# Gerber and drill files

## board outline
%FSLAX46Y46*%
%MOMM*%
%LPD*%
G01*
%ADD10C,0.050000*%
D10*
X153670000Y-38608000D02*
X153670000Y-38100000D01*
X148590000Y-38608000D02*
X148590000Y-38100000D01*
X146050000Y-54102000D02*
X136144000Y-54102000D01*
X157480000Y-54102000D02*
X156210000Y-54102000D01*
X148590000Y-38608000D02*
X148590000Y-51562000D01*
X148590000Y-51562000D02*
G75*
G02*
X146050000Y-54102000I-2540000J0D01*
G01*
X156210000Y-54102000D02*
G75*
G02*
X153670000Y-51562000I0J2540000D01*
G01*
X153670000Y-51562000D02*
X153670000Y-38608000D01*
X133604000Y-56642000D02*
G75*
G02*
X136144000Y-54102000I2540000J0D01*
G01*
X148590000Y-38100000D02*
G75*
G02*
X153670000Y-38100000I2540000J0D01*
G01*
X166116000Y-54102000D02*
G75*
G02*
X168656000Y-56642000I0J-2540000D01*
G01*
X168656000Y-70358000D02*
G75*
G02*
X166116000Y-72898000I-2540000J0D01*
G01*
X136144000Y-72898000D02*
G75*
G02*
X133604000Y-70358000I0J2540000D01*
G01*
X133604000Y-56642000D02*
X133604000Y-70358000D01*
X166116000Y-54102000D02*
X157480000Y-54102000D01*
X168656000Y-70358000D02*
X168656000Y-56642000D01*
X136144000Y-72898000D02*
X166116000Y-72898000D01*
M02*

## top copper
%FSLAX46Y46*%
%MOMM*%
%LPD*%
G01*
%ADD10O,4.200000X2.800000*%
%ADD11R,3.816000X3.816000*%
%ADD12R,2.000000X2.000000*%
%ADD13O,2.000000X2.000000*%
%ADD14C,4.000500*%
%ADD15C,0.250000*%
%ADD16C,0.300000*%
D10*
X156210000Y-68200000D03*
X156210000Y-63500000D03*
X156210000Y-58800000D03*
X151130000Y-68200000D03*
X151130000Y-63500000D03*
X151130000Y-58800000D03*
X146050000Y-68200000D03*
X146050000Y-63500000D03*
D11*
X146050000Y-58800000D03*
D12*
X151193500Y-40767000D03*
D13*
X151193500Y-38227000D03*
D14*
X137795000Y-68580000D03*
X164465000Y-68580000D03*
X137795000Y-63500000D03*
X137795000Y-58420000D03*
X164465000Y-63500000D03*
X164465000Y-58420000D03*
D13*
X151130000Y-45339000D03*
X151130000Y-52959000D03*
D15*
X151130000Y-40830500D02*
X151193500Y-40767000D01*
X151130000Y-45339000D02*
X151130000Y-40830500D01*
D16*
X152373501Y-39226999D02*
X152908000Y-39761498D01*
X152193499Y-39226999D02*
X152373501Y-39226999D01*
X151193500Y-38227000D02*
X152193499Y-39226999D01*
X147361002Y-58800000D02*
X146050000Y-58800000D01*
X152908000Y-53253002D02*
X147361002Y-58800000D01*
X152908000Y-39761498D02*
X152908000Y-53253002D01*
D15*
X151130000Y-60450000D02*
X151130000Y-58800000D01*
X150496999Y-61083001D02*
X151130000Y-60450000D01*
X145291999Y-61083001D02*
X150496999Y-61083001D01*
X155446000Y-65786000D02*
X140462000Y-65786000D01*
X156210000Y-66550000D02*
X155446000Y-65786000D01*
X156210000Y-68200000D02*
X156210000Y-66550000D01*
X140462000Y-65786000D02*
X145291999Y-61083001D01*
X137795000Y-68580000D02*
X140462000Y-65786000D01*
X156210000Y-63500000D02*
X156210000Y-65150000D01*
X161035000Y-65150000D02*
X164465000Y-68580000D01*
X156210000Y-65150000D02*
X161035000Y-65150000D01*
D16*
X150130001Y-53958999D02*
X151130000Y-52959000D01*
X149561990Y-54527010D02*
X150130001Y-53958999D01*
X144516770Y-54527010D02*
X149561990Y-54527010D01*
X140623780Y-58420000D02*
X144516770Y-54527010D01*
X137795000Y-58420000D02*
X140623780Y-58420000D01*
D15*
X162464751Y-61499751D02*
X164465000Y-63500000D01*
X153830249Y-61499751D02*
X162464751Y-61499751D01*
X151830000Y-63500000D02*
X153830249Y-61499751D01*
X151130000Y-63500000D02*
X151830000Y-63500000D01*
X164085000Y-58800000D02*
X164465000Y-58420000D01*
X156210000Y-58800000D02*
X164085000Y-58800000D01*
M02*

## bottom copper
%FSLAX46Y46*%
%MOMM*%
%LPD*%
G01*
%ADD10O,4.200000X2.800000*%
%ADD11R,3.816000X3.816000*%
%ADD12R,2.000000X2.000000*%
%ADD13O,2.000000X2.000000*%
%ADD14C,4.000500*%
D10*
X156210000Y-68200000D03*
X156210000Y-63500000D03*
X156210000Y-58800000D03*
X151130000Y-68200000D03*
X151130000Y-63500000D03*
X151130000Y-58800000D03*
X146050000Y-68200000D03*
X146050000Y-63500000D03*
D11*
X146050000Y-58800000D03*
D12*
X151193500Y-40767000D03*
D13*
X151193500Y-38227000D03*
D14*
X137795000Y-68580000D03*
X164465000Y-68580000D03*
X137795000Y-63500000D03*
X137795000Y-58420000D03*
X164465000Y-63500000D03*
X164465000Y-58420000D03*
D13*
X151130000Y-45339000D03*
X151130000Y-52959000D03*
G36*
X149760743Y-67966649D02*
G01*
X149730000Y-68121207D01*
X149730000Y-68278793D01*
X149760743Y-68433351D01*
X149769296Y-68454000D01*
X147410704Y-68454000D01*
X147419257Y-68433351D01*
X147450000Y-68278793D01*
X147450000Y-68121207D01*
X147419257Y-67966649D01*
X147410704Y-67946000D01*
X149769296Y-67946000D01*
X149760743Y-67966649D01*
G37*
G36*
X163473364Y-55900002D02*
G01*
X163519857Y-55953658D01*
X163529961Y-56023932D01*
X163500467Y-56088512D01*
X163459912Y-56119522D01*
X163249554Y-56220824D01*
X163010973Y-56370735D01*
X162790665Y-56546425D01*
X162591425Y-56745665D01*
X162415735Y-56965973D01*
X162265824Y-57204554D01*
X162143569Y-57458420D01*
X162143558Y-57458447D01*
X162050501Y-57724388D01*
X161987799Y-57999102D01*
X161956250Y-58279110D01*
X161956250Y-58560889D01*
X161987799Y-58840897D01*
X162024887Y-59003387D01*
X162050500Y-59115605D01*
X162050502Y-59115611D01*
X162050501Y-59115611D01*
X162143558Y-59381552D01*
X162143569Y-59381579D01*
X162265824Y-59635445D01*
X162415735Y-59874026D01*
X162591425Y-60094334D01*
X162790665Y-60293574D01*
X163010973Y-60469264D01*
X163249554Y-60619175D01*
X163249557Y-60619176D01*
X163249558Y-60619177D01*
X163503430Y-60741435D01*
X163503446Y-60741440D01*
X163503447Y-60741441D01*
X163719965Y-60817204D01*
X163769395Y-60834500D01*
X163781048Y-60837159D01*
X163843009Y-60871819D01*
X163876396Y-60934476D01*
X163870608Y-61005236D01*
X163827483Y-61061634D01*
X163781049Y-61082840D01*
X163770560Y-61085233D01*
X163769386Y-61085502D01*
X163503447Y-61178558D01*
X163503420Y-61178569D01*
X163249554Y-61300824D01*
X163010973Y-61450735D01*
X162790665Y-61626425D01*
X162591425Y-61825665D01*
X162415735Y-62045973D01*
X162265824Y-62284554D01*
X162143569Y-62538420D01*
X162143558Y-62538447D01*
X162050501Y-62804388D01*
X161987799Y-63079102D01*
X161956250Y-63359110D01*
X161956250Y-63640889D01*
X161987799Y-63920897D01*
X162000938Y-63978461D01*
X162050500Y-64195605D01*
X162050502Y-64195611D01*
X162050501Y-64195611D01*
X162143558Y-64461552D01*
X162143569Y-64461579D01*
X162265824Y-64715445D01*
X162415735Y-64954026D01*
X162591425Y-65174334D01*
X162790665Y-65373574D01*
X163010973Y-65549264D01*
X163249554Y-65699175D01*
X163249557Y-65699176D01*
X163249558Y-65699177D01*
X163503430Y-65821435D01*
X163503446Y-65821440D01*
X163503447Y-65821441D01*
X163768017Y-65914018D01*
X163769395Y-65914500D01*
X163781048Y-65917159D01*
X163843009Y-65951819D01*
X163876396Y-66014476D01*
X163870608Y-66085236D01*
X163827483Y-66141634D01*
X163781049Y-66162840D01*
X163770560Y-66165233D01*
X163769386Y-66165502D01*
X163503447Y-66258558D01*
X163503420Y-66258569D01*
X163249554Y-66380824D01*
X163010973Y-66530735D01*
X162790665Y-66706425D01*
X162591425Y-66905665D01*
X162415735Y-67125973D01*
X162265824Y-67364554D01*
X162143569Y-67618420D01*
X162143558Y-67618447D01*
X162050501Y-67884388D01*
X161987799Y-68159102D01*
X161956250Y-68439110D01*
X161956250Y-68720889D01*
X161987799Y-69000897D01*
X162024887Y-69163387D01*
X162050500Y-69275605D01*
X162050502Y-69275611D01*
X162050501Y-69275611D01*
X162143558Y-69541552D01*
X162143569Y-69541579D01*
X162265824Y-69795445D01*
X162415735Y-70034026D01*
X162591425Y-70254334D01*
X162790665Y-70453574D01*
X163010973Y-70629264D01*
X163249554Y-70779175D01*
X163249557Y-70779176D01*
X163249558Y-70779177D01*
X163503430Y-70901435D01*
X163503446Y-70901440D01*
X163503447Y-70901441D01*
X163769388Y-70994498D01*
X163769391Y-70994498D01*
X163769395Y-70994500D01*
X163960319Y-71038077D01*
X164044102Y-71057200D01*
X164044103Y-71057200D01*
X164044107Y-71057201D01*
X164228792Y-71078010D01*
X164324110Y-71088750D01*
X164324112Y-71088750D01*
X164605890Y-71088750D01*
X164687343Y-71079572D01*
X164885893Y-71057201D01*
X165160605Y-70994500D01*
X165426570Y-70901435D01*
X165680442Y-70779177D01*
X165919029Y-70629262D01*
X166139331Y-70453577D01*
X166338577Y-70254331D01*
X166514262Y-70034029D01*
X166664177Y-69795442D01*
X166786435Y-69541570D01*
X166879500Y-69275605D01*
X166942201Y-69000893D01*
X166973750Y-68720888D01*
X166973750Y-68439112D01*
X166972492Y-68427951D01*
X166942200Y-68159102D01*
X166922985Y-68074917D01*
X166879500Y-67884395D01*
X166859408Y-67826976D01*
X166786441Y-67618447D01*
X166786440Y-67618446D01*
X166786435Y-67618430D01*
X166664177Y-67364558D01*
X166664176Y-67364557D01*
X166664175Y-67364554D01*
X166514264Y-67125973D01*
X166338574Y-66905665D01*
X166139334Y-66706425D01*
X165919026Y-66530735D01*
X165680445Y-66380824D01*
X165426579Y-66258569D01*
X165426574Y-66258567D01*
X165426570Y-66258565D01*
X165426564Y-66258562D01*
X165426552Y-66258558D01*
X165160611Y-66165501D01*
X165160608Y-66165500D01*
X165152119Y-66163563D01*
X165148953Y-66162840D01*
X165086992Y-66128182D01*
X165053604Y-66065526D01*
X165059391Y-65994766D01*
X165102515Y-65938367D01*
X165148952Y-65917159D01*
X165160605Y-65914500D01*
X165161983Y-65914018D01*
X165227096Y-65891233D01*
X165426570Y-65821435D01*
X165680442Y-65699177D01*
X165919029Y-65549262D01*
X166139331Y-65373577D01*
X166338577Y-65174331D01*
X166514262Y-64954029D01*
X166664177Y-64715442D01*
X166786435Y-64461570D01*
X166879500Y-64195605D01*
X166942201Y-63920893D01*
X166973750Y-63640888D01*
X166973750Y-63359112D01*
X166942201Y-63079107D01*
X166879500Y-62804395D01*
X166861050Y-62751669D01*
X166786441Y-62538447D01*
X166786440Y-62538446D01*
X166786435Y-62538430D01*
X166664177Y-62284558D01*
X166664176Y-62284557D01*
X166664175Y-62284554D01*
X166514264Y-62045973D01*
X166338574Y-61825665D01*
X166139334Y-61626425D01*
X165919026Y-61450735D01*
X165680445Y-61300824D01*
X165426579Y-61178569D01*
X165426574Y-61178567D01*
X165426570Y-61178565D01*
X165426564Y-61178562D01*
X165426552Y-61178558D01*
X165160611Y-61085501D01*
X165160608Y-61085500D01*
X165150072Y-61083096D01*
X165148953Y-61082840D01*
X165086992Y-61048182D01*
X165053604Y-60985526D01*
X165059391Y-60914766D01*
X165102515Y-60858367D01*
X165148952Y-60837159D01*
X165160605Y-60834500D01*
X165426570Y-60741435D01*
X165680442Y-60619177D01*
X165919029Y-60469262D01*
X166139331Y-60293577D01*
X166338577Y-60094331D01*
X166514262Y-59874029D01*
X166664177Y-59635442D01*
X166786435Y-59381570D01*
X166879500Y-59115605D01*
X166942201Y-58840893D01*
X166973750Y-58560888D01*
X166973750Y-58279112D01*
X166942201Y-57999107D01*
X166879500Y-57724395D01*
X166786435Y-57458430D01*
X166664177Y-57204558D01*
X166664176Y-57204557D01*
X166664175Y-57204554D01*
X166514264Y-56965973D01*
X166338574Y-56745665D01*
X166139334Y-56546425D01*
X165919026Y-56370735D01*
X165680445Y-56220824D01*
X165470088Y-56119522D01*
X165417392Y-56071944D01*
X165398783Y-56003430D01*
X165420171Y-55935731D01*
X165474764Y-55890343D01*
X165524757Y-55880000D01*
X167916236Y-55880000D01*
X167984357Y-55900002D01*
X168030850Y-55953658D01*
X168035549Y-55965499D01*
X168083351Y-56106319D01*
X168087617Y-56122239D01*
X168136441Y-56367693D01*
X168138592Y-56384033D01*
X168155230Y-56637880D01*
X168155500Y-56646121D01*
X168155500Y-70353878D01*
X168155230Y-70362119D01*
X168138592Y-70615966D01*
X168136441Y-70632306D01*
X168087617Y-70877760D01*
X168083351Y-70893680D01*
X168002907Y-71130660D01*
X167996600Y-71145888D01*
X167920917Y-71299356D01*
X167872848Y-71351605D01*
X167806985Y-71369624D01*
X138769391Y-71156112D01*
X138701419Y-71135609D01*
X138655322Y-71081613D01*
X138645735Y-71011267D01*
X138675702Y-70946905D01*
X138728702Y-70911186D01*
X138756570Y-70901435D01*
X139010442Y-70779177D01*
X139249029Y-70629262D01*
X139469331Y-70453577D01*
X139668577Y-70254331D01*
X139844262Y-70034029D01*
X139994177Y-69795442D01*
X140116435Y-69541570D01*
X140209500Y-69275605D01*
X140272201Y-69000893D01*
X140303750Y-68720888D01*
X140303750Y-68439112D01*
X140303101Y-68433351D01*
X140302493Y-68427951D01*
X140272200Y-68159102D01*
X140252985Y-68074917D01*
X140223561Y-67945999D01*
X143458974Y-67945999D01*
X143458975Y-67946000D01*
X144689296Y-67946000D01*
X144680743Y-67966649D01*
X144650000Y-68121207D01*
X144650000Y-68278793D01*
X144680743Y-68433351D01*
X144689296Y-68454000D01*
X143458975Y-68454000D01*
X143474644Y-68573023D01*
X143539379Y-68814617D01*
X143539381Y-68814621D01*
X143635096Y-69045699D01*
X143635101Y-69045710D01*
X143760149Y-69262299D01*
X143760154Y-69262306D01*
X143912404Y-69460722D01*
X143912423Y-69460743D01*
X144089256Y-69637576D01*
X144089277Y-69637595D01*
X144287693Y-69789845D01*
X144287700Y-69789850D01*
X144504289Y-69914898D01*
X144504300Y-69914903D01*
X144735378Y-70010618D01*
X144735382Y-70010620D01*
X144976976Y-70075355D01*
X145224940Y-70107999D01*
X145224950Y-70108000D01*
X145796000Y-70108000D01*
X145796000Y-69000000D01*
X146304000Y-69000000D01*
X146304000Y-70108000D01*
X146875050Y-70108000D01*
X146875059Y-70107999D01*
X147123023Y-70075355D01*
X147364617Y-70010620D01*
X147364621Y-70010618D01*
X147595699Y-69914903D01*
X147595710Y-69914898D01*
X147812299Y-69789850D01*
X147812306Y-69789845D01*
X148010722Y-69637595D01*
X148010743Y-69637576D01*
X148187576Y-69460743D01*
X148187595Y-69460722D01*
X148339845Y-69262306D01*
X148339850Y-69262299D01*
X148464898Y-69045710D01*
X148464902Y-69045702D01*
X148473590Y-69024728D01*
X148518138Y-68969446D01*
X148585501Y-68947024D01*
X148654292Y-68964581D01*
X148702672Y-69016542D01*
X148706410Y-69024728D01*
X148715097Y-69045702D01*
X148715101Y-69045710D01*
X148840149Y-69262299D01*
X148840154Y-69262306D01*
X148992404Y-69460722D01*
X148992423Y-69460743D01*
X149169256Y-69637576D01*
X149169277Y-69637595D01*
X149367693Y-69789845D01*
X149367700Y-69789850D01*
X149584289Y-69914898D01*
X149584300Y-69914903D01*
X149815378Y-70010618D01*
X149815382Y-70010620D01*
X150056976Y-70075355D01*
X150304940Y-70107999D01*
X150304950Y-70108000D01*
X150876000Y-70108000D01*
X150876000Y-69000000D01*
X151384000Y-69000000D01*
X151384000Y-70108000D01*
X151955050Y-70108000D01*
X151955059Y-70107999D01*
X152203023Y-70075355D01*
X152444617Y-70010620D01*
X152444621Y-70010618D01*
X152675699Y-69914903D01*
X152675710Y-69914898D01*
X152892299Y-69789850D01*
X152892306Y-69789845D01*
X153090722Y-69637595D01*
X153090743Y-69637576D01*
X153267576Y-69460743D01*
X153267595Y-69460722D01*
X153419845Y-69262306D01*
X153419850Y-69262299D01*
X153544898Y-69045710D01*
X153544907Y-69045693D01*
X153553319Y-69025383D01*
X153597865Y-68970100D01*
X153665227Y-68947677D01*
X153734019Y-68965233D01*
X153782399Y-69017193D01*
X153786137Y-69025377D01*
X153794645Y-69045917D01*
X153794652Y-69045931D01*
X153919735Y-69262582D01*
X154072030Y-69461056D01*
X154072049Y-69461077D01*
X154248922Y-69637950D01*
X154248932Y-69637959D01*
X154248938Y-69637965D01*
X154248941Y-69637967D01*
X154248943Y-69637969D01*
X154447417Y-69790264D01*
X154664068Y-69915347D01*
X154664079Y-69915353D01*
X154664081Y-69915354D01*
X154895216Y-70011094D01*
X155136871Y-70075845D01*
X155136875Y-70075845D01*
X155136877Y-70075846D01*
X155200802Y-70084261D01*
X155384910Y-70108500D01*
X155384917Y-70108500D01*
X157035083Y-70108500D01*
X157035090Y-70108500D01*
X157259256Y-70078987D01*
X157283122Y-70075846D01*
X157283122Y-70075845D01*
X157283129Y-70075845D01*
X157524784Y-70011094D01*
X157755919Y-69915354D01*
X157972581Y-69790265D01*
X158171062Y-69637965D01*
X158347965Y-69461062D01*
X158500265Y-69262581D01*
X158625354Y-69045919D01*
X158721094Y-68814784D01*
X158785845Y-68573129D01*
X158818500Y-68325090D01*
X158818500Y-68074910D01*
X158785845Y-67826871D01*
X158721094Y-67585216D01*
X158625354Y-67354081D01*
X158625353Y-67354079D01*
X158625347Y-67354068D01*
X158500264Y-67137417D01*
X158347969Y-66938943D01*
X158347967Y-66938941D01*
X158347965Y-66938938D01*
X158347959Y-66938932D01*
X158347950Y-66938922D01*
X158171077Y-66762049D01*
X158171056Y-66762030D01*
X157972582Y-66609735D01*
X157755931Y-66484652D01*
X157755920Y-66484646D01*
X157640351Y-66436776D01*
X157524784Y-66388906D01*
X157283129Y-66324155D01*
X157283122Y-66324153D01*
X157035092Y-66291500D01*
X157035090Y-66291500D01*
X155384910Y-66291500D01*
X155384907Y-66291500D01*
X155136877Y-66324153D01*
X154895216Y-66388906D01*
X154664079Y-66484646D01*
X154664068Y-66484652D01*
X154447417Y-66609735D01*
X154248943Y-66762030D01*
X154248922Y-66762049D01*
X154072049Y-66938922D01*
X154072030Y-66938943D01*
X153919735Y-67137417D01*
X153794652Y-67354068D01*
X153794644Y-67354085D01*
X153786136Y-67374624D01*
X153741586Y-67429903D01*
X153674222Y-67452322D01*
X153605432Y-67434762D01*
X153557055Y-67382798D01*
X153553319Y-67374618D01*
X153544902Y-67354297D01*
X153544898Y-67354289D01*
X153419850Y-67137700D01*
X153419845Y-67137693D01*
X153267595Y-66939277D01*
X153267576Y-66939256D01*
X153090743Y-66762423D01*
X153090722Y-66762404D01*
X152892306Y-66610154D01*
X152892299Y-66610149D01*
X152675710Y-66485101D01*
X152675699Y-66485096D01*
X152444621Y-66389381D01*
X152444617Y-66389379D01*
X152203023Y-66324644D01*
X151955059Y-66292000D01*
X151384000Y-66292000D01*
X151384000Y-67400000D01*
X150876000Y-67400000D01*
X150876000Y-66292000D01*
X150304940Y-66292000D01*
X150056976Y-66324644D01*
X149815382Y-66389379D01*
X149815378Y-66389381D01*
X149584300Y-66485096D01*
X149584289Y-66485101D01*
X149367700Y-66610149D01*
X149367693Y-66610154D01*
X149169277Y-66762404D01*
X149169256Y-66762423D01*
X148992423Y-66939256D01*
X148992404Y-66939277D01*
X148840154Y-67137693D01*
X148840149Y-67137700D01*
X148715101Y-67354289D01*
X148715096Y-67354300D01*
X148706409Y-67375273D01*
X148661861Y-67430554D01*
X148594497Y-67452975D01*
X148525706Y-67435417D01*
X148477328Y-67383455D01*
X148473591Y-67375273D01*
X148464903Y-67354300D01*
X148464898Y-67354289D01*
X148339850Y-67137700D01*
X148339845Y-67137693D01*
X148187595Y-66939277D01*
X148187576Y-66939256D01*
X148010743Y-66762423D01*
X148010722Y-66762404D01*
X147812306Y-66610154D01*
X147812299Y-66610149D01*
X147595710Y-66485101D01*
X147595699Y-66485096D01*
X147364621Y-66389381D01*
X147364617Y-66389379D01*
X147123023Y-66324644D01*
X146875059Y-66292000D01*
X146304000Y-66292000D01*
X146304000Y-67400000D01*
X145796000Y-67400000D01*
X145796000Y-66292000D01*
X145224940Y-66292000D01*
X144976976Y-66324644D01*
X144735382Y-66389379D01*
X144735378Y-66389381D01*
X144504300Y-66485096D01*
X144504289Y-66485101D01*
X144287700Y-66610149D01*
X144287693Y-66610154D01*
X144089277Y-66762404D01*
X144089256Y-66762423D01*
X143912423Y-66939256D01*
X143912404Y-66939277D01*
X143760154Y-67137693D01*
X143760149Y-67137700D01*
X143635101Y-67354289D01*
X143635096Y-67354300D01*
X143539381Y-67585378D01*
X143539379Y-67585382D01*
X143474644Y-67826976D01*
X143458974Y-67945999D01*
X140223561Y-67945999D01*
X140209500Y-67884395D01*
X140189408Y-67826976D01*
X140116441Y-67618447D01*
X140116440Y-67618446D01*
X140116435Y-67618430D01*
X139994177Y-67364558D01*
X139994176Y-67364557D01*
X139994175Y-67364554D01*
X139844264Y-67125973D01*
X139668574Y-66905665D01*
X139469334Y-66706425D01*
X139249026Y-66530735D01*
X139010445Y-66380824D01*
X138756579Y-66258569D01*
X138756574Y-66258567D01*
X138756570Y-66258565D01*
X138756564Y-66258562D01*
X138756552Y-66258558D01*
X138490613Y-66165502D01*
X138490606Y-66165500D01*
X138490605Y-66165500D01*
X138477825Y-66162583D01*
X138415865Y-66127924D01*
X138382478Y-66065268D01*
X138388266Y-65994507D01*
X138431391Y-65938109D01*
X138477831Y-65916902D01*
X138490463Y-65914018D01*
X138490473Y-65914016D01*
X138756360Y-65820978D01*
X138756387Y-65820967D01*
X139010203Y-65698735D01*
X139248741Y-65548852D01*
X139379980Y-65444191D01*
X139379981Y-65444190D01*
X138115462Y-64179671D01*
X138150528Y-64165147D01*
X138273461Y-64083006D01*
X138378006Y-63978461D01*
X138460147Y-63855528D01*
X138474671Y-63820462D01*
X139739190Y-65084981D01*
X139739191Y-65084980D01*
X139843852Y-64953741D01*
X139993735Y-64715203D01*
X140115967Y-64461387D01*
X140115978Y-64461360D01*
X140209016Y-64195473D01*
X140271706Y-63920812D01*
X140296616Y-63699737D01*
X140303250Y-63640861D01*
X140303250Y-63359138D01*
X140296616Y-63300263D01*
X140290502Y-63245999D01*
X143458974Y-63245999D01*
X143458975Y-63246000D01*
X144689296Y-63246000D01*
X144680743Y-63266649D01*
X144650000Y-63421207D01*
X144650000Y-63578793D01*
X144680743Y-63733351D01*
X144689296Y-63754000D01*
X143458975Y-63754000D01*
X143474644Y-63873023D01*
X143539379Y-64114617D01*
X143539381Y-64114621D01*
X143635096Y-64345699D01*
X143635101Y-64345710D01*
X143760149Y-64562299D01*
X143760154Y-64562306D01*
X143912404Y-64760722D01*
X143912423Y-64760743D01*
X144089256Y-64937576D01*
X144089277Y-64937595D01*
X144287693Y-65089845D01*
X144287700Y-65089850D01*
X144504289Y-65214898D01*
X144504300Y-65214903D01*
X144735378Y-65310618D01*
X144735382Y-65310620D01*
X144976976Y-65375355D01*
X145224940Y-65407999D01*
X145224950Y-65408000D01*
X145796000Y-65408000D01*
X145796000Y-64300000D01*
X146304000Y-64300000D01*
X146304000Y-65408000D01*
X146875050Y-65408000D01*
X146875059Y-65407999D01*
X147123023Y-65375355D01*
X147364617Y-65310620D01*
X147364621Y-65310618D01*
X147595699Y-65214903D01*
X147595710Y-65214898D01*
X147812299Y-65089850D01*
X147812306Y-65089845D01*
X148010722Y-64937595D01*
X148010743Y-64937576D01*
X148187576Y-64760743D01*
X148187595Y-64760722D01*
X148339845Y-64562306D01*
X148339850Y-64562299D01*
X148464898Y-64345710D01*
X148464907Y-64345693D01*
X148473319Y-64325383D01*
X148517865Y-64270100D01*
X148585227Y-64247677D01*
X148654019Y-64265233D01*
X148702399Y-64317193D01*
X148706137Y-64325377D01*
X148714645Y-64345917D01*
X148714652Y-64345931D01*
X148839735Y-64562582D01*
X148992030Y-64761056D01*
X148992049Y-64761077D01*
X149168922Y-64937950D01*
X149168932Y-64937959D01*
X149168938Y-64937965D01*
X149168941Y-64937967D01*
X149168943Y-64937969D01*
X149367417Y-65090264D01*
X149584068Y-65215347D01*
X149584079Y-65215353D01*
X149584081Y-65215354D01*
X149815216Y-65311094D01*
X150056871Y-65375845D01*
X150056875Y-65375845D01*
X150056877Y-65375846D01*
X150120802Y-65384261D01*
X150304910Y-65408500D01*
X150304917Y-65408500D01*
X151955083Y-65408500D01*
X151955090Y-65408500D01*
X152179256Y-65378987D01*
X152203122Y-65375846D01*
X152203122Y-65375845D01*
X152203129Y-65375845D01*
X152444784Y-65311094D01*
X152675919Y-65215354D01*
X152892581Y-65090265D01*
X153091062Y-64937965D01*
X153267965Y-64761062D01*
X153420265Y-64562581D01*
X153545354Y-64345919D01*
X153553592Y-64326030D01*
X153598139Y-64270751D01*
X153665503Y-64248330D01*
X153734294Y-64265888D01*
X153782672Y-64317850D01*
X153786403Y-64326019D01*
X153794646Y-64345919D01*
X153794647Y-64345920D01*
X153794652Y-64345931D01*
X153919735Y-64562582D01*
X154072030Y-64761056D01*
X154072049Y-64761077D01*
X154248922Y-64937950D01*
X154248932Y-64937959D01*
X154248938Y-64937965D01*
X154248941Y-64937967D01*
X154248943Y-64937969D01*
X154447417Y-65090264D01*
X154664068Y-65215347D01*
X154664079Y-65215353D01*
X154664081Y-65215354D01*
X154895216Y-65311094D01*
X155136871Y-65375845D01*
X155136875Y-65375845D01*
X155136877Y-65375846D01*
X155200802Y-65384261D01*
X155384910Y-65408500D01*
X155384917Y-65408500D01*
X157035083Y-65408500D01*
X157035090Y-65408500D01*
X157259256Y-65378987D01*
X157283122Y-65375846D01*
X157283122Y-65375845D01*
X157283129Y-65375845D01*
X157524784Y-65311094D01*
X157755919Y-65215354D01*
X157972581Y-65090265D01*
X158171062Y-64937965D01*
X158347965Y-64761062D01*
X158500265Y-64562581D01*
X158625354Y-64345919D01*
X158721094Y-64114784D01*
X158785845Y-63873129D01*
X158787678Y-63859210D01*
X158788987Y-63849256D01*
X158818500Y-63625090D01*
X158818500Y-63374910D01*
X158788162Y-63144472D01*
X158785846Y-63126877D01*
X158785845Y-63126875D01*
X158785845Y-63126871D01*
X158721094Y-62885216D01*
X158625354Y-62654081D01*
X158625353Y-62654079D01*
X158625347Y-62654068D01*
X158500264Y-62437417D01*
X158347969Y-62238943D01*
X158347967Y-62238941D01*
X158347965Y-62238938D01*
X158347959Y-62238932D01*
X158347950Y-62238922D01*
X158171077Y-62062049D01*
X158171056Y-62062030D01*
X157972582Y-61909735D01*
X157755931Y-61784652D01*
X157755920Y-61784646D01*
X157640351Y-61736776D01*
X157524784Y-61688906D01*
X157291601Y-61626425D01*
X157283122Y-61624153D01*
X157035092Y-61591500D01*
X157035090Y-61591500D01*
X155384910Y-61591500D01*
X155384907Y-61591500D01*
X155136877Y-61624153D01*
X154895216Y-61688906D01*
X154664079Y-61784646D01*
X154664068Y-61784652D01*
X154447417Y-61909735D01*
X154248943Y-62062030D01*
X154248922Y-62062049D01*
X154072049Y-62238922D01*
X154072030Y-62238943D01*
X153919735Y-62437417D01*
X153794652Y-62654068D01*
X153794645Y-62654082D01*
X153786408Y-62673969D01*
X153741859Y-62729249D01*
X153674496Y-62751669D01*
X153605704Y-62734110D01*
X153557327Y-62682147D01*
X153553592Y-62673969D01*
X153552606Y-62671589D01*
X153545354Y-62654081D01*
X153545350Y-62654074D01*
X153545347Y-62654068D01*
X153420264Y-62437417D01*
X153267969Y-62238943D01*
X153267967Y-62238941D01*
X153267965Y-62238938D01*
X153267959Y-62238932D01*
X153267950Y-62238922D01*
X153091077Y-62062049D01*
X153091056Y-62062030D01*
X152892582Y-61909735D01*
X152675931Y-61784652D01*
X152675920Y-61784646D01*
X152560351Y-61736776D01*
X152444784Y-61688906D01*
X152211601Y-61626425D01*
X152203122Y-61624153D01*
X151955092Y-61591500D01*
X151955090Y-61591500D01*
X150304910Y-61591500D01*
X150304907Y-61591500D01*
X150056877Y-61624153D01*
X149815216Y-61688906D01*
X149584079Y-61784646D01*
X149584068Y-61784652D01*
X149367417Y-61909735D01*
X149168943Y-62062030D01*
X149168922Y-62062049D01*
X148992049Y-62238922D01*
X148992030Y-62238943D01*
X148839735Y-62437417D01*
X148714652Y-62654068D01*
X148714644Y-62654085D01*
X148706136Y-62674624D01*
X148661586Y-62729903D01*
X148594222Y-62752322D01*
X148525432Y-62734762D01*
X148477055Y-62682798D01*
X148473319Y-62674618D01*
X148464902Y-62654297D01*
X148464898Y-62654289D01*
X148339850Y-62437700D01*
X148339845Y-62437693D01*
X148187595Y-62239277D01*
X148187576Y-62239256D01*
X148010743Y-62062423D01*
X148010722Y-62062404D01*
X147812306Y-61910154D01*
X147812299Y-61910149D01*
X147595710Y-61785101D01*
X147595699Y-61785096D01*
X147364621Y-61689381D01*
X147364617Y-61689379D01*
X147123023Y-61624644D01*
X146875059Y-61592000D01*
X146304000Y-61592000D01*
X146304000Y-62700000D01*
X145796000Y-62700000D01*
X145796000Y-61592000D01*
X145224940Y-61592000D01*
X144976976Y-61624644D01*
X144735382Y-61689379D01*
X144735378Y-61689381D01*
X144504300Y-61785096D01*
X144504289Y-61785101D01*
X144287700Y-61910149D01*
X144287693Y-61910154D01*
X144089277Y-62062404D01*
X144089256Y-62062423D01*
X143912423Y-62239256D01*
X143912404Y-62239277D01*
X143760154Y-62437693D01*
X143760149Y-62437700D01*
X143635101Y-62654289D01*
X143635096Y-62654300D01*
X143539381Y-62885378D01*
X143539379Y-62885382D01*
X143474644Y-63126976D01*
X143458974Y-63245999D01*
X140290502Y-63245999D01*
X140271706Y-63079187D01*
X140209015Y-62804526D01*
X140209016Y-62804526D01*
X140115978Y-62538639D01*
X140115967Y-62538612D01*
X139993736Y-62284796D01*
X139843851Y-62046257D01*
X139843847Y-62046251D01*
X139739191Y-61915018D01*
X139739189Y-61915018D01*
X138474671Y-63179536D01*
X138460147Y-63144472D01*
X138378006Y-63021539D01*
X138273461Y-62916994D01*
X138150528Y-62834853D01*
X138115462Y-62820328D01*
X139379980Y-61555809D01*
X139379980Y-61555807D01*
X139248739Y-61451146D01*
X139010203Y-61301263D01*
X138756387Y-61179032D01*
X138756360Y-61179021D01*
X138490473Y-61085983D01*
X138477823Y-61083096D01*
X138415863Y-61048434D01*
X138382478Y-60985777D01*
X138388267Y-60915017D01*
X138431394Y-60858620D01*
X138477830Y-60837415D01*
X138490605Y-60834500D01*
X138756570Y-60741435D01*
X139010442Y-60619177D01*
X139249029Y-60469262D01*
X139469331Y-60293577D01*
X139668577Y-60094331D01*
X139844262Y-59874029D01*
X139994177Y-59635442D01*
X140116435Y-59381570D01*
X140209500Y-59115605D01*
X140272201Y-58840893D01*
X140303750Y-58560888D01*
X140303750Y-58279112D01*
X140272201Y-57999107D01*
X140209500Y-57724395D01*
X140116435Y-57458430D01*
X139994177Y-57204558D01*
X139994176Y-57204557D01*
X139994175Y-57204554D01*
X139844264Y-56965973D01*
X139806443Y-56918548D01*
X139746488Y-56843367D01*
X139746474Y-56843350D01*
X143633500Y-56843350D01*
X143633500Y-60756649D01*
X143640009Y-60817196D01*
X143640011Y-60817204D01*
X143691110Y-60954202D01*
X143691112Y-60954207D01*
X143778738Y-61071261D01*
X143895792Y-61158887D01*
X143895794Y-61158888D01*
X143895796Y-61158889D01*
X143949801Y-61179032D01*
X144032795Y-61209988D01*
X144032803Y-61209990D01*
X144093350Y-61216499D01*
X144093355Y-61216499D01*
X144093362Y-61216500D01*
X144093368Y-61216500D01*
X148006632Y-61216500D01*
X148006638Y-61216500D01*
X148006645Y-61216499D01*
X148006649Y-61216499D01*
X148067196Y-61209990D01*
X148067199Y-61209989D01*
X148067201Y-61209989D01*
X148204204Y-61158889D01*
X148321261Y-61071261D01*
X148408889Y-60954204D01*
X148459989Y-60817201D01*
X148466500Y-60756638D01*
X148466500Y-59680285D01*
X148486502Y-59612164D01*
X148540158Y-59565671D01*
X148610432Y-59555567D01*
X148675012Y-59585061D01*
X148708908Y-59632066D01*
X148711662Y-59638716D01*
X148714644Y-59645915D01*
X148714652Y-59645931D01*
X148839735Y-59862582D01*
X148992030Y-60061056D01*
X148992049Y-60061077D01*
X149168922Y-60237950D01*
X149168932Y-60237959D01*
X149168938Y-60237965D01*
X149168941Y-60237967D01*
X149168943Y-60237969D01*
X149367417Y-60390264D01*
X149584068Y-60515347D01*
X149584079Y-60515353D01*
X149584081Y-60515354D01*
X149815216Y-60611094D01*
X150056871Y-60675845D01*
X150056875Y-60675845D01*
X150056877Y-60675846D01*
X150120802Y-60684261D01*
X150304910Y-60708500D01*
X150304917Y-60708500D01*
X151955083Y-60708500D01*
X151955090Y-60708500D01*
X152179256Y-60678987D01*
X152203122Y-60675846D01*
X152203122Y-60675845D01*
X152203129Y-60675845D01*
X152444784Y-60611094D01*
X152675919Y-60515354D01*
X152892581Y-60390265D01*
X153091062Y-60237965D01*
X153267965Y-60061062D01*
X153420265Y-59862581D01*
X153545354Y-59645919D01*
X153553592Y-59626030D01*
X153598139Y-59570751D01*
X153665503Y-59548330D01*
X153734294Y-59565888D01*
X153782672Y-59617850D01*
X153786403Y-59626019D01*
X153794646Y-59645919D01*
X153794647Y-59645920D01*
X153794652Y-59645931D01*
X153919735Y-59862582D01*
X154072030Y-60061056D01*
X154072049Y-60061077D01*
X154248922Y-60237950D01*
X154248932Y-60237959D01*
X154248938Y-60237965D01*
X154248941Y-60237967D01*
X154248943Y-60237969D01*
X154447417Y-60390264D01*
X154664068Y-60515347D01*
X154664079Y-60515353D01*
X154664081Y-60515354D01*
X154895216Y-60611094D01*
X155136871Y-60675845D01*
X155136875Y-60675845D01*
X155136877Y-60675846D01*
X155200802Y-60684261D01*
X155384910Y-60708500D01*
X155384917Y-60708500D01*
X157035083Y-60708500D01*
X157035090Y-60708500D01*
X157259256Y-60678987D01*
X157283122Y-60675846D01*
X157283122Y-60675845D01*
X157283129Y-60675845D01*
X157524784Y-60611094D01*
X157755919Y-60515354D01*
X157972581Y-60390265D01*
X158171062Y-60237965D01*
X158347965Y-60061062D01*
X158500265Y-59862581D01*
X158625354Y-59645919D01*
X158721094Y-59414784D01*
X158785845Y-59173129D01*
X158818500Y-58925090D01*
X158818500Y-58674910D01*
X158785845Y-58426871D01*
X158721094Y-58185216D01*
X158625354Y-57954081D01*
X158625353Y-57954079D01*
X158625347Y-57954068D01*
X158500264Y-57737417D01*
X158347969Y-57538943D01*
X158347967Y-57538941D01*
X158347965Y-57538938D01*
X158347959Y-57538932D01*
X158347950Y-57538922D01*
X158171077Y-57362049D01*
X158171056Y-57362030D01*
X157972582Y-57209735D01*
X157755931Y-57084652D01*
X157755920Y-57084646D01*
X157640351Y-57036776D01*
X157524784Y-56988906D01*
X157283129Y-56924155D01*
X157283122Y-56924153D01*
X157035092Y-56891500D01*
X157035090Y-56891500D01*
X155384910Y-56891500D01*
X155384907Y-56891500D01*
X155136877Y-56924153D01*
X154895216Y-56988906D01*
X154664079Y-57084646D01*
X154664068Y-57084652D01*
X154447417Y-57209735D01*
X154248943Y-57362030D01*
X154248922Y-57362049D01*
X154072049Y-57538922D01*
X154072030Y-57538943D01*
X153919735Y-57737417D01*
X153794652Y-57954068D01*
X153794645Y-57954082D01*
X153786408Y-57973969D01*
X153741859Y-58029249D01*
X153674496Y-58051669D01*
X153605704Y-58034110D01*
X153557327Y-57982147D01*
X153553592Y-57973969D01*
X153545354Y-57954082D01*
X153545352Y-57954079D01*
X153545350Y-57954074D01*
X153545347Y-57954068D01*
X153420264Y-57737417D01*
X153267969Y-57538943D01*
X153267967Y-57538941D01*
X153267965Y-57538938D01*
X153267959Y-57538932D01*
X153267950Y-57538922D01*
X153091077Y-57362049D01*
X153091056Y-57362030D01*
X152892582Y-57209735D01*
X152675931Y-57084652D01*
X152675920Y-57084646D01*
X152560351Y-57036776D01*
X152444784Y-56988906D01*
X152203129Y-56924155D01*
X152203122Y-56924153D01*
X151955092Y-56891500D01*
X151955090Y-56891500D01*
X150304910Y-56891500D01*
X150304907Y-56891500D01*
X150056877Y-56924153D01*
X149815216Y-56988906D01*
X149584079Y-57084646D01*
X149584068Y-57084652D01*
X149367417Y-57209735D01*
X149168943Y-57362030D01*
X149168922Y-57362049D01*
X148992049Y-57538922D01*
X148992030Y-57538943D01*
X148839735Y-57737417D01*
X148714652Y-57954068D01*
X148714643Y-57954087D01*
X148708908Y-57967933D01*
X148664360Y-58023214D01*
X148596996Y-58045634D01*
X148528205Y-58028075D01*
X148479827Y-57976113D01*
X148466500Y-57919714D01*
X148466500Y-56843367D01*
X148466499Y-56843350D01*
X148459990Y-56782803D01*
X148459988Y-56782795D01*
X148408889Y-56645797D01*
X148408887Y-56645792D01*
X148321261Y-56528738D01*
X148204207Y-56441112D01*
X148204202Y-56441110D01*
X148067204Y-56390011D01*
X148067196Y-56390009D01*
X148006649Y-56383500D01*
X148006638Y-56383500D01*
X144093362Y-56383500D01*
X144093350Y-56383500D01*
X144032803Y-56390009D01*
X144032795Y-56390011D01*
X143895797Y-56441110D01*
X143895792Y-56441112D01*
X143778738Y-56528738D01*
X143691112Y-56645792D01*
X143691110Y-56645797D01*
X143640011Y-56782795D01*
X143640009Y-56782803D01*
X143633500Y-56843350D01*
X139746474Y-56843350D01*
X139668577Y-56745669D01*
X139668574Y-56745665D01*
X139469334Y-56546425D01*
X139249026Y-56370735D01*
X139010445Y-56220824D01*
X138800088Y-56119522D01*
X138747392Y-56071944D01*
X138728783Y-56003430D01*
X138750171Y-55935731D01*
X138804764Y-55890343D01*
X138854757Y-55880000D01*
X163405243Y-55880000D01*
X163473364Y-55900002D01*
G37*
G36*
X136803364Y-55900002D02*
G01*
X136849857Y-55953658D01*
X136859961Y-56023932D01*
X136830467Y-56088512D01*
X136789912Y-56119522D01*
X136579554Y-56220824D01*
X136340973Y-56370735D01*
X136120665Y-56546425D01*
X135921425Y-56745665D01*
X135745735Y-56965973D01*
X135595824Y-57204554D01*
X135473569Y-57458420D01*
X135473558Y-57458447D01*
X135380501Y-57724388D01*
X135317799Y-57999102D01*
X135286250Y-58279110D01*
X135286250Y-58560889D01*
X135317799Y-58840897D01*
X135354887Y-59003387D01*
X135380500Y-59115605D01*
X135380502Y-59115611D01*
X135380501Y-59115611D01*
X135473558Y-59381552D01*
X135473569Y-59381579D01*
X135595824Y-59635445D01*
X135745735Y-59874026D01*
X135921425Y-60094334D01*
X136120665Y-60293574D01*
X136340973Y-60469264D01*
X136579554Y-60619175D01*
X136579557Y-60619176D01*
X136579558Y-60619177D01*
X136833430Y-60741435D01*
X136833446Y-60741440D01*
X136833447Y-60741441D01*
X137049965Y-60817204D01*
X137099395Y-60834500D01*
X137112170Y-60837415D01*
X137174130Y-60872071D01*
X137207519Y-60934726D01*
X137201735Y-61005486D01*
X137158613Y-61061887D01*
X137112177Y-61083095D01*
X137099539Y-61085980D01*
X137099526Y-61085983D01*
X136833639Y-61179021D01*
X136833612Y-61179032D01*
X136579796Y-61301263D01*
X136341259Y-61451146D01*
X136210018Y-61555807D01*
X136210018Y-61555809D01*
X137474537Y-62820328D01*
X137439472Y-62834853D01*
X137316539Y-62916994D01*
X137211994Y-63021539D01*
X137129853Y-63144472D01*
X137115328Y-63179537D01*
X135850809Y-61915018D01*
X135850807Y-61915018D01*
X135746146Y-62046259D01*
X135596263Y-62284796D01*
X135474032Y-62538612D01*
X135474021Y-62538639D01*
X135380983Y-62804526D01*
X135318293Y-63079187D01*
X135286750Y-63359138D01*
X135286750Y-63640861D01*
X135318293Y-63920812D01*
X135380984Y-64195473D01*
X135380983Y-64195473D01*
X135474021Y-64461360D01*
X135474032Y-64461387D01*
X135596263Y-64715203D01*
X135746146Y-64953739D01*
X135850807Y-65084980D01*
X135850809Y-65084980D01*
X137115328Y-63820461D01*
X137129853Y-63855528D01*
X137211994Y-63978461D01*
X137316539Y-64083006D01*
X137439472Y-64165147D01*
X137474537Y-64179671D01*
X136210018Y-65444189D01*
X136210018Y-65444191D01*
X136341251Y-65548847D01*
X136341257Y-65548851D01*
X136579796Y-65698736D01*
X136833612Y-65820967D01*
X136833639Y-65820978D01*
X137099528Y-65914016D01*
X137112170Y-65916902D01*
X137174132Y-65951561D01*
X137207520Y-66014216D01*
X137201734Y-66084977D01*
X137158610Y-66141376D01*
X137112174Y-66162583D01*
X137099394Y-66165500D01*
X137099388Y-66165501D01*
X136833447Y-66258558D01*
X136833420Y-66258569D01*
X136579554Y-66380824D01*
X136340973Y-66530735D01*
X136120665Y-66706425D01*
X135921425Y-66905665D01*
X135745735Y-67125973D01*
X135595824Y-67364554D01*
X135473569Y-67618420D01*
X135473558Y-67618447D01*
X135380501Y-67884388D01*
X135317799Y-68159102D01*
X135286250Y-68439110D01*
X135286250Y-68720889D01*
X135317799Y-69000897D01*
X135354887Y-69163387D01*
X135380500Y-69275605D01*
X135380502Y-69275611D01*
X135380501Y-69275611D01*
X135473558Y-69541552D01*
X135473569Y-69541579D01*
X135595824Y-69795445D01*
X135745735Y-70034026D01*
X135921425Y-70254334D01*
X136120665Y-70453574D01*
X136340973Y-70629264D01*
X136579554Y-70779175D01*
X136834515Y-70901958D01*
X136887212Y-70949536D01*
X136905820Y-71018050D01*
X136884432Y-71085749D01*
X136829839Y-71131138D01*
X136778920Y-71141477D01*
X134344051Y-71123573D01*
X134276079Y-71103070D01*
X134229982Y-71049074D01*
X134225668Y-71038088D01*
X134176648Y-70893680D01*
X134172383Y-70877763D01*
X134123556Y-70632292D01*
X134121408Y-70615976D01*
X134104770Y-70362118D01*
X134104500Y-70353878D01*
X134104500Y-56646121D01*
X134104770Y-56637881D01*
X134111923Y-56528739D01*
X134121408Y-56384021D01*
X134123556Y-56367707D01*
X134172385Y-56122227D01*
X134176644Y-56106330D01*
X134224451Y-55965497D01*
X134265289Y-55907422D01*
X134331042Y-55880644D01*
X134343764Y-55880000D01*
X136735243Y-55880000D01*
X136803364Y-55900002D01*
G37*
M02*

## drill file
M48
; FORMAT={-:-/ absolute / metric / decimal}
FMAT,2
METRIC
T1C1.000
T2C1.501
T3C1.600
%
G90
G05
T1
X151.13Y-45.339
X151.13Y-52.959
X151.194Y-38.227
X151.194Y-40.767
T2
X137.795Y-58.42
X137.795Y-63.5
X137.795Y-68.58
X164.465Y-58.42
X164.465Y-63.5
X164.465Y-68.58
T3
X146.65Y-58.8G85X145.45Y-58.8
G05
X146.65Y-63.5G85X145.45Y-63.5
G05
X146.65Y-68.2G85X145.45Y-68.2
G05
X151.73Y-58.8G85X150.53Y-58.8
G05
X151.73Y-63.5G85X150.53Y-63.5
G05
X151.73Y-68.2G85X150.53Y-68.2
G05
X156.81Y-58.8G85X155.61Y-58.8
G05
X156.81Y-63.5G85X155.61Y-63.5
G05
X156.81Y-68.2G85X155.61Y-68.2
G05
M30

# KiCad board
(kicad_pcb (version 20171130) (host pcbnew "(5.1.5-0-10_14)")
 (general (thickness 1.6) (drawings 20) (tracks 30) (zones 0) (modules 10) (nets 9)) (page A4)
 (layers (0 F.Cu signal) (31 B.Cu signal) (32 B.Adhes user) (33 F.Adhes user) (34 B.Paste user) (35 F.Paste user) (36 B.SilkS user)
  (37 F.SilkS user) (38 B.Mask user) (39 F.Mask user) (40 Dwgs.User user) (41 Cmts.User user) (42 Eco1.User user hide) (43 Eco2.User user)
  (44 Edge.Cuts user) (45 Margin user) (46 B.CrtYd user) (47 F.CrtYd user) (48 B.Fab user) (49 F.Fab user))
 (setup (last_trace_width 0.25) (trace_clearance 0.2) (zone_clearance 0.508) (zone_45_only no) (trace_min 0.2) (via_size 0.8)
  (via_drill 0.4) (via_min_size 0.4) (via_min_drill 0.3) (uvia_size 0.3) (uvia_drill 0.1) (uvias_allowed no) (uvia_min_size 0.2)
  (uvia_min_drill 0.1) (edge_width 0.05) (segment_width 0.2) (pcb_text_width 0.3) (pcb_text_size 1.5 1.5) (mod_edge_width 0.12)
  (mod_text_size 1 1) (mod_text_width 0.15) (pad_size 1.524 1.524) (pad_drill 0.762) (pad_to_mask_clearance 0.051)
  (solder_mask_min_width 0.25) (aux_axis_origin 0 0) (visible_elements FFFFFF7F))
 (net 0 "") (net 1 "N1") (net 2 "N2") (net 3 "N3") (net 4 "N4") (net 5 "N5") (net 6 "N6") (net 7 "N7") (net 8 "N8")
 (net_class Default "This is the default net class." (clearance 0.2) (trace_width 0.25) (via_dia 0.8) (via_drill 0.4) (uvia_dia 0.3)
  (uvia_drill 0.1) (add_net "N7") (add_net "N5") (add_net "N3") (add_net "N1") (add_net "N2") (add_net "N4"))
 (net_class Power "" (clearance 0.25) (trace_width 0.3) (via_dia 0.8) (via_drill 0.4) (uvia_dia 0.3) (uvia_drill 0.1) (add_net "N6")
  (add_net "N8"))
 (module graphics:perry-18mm (layer F.Cu) (at 151.13 62.23)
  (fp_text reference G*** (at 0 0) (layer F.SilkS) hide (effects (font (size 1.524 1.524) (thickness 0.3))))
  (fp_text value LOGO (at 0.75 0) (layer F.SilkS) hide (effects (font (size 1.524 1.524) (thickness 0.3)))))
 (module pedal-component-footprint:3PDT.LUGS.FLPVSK (layer F.Cu) (at 151.13 63.5)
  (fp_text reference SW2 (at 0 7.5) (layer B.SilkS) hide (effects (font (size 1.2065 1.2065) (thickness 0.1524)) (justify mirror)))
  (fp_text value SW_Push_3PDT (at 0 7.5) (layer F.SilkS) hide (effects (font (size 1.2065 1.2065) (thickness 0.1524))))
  (pad 9 thru_hole oval (at 5.08 4.7 180) (size 4.2 2.8) (drill oval 2.8 1.6) (layers *.Cu *.Mask) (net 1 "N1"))
  (pad 8 thru_hole oval (at 5.08 0 180) (size 4.2 2.8) (drill oval 2.8 1.6) (layers *.Cu *.Mask) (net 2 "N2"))
  (pad 7 thru_hole oval (at 5.08 -4.7 180) (size 4.2 2.8) (drill oval 2.8 1.6) (layers *.Cu *.Mask) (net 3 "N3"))
  (pad 6 thru_hole oval (at 0 4.7 180) (size 4.2 2.8) (drill oval 2.8 1.6) (layers *.Cu *.Mask) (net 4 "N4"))
  (pad 5 thru_hole oval (at 0 0 180) (size 4.2 2.8) (drill oval 2.8 1.6) (layers *.Cu *.Mask) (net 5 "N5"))
  (pad 4 thru_hole oval (at 0 -4.7 180) (size 4.2 2.8) (drill oval 2.8 1.6) (layers *.Cu *.Mask) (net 1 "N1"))
  (pad 3 thru_hole oval (at -5.08 4.7 180) (size 4.2 2.8) (drill oval 2.8 1.6) (layers *.Cu *.Mask) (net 4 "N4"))
  (pad 2 thru_hole oval (at -5.08 0 180) (size 4.2 2.8) (drill oval 2.8 1.6) (layers *.Cu *.Mask) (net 4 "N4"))
  (pad 1 thru_hole rect (at -5.08 -4.7 180) (size 3.816 3.816) (drill oval 2.8 1.6) (layers *.Cu *.Mask) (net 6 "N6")))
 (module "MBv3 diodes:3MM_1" (layer F.Cu) (at 151.1935 39.497 90)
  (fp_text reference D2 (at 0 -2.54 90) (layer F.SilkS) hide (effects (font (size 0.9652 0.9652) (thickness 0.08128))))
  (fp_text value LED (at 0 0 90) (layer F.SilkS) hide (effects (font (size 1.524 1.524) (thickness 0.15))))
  (pad 2 thru_hole rect (at -1.27 0 90) (size 2 2) (drill 1) (layers *.Cu *.Mask) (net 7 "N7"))
  (pad 1 thru_hole oval (at 1.27 0 90) (size 2 2) (drill 1) (layers *.Cu *.Mask) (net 6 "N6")))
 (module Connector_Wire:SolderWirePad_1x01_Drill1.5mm (layer F.Cu) (at 137.795 68.58 270)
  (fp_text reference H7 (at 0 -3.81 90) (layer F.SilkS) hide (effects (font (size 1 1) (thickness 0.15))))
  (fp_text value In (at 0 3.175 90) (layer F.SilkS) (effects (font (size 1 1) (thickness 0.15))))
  (pad 1 thru_hole circle (at 0 0 270) (size 4.0005 4.0005) (drill 1.50114) (layers *.Cu *.Mask) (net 1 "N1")))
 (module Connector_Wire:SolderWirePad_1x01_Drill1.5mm (layer F.Cu) (at 164.465 68.58 90)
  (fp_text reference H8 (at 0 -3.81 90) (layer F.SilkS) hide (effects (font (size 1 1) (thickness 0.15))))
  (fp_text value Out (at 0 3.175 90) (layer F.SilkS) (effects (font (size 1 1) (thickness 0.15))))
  (pad 1 thru_hole circle (at 0 0 90) (size 4.0005 4.0005) (drill 1.50114) (layers *.Cu *.Mask) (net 2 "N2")))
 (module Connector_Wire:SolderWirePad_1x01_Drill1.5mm (layer F.Cu) (at 137.795 63.5 270)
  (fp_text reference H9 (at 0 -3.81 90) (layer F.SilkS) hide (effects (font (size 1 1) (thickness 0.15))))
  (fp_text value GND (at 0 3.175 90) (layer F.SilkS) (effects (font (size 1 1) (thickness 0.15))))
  (pad 1 thru_hole circle (at 0 0 270) (size 4.0005 4.0005) (drill 1.50114) (layers *.Cu *.Mask) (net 4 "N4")))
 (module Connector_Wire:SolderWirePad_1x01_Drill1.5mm (layer F.Cu) (at 137.795 58.42 270)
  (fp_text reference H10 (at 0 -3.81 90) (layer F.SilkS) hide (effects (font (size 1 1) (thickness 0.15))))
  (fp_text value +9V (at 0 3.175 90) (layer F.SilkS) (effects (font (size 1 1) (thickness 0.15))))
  (pad 1 thru_hole circle (at 0 0 270) (size 4.0005 4.0005) (drill 1.50114) (layers *.Cu *.Mask) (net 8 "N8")))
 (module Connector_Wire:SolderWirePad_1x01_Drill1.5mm (layer F.Cu) (at 164.465 63.5 90)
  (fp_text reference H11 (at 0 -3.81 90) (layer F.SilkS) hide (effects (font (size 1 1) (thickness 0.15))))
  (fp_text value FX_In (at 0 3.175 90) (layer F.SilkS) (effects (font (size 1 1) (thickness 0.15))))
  (pad 1 thru_hole circle (at 0 0 90) (size 4.0005 4.0005) (drill 1.50114) (layers *.Cu *.Mask) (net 5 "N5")))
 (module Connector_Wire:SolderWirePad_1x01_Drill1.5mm (layer F.Cu) (at 164.465 58.42 90)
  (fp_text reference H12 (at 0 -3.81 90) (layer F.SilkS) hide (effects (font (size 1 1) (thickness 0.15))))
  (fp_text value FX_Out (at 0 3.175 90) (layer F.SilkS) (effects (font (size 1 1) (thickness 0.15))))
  (pad 1 thru_hole circle (at 0 0 90) (size 4.0005 4.0005) (drill 1.50114) (layers *.Cu *.Mask) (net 3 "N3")))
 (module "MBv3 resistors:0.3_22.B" (layer F.Cu) (at 151.13 49.149 270)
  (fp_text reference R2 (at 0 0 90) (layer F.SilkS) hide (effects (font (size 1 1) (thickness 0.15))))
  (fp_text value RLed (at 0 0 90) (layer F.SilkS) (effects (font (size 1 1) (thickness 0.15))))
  (pad 1 thru_hole oval (at -3.81 0 270) (size 2 2) (drill 1) (layers *.Cu *.Mask) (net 7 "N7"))
  (pad 2 thru_hole oval (at 3.81 0 270) (size 2 2) (drill 1) (layers *.Cu *.Mask) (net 8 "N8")))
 (gr_line (start 153.67 38.608) (end 153.67 38.1) (layer Edge.Cuts) (width 0.05))
 (gr_line (start 148.59 38.608) (end 148.59 38.1) (layer Edge.Cuts) (width 0.05))
 (gr_line (start 146.05 54.102) (end 136.144 54.102) (layer Edge.Cuts) (width 0.05))
 (gr_line (start 157.48 54.102) (end 156.21 54.102) (layer Edge.Cuts) (width 0.05))
 (gr_line (start 148.59 38.608) (end 148.59 51.562) (layer Edge.Cuts) (width 0.05))
 (gr_arc (start 146.05 51.562) (end 146.05 54.102) (angle -90) (layer Edge.Cuts) (width 0.05))
 (gr_arc (start 156.21 51.562) (end 153.67 51.562) (angle -90) (layer Edge.Cuts) (width 0.05))
 (gr_line (start 153.67 51.562) (end 153.67 38.608) (layer Edge.Cuts) (width 0.05))
 (gr_arc (start 136.144 56.642) (end 136.144 54.102) (angle -90) (layer Edge.Cuts) (width 0.05))
 (gr_arc (start 151.13 38.1) (end 153.67 38.1) (angle -180) (layer Edge.Cuts) (width 0.05))
 (gr_arc (start 166.116 56.642) (end 168.656 56.642) (angle -90) (layer Edge.Cuts) (width 0.05))
 (gr_arc (start 166.116 70.358) (end 166.116 72.898) (angle -90) (layer Edge.Cuts) (width 0.05))
 (gr_arc (start 136.144 70.358) (end 133.604 70.358) (angle -90) (layer Edge.Cuts) (width 0.05))
 (gr_line (start 133.604 56.642) (end 133.604 70.358) (layer Edge.Cuts) (width 0.05))
 (gr_line (start 166.116 54.102) (end 157.48 54.102) (layer Edge.Cuts) (width 0.05))
 (gr_line (start 168.656 70.358) (end 168.656 56.642) (layer Edge.Cuts) (width 0.05))
 (gr_line (start 136.144 72.898) (end 166.116 72.898) (layer Edge.Cuts) (width 0.05))
 (segment (start 151.13 40.8305) (end 151.1935 40.767) (width 0.25) (layer F.Cu) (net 7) (status 30))
 (segment (start 151.13 45.339) (end 151.13 40.8305) (width 0.25) (layer F.Cu) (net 7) (status 30))
 (segment (start 152.373501 39.226999) (end 152.908 39.761498) (width 0.3) (layer F.Cu) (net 6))
 (segment (start 152.193499 39.226999) (end 152.373501 39.226999) (width 0.3) (layer F.Cu) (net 6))
 (segment (start 151.1935 38.227) (end 152.193499 39.226999) (width 0.3) (layer F.Cu) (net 6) (status 10))
 (segment (start 147.361002 58.8) (end 146.05 58.8) (width 0.3) (layer F.Cu) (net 6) (status 30))
 (segment (start 152.908 53.253002) (end 147.361002 58.8) (width 0.3) (layer F.Cu) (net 6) (status 20))
 (segment (start 152.908 39.761498) (end 152.908 53.253002) (width 0.3) (layer F.Cu) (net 6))
 (segment (start 151.13 60.45) (end 151.13 58.8) (width 0.25) (layer F.Cu) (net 1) (status 20))
 (segment (start 150.496999 61.083001) (end 151.13 60.45) (width 0.25) (layer F.Cu) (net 1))
 (segment (start 145.291999 61.083001) (end 150.496999 61.083001) (width 0.25) (layer F.Cu) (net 1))
 (segment (start 155.446 65.786) (end 140.462 65.786) (width 0.25) (layer F.Cu) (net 1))
 (segment (start 156.21 66.55) (end 155.446 65.786) (width 0.25) (layer F.Cu) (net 1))
 (segment (start 156.21 68.2) (end 156.21 66.55) (width 0.25) (layer F.Cu) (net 1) (status 10))
 (segment (start 140.462 65.786) (end 145.291999 61.083001) (width 0.25) (layer F.Cu) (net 1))
 (segment (start 137.795 68.58) (end 140.462 65.786) (width 0.25) (layer F.Cu) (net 1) (status 10))
 (segment (start 156.21 63.5) (end 156.21 65.15) (width 0.25) (layer F.Cu) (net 2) (status 10))
 (segment (start 161.035 65.15) (end 164.465 68.58) (width 0.25) (layer F.Cu) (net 2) (status 20))
 (segment (start 156.21 65.15) (end 161.035 65.15) (width 0.25) (layer F.Cu) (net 2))
 (segment (start 150.130001 53.958999) (end 151.13 52.959) (width 0.3) (layer F.Cu) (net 8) (status 20))
 (segment (start 149.56199 54.52701) (end 150.130001 53.958999) (width 0.3) (layer F.Cu) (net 8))
 (segment (start 144.51677 54.52701) (end 149.56199 54.52701) (width 0.3) (layer F.Cu) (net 8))
 (segment (start 140.62378 58.42) (end 144.51677 54.52701) (width 0.3) (layer F.Cu) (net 8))
 (segment (start 137.795 58.42) (end 140.62378 58.42) (width 0.3) (layer F.Cu) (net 8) (status 10))
 (segment (start 162.464751 61.499751) (end 164.465 63.5) (width 0.25) (layer F.Cu) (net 5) (status 20))
 (segment (start 153.830249 61.499751) (end 162.464751 61.499751) (width 0.25) (layer F.Cu) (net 5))
 (segment (start 151.83 63.5) (end 153.830249 61.499751) (width 0.25) (layer F.Cu) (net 5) (status 10))
 (segment (start 151.13 63.5) (end 151.83 63.5) (width 0.25) (layer F.Cu) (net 5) (status 30))
 (segment (start 164.085 58.8) (end 164.465 58.42) (width 0.25) (layer F.Cu) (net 3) (status 30))
 (segment (start 156.21 58.8) (end 164.085 58.8) (width 0.25) (layer F.Cu) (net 3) (status 30))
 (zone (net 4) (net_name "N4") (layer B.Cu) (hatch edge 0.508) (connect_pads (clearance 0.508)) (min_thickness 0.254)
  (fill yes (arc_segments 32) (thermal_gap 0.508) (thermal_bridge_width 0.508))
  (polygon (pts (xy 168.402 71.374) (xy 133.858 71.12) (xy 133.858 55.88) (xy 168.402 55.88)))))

